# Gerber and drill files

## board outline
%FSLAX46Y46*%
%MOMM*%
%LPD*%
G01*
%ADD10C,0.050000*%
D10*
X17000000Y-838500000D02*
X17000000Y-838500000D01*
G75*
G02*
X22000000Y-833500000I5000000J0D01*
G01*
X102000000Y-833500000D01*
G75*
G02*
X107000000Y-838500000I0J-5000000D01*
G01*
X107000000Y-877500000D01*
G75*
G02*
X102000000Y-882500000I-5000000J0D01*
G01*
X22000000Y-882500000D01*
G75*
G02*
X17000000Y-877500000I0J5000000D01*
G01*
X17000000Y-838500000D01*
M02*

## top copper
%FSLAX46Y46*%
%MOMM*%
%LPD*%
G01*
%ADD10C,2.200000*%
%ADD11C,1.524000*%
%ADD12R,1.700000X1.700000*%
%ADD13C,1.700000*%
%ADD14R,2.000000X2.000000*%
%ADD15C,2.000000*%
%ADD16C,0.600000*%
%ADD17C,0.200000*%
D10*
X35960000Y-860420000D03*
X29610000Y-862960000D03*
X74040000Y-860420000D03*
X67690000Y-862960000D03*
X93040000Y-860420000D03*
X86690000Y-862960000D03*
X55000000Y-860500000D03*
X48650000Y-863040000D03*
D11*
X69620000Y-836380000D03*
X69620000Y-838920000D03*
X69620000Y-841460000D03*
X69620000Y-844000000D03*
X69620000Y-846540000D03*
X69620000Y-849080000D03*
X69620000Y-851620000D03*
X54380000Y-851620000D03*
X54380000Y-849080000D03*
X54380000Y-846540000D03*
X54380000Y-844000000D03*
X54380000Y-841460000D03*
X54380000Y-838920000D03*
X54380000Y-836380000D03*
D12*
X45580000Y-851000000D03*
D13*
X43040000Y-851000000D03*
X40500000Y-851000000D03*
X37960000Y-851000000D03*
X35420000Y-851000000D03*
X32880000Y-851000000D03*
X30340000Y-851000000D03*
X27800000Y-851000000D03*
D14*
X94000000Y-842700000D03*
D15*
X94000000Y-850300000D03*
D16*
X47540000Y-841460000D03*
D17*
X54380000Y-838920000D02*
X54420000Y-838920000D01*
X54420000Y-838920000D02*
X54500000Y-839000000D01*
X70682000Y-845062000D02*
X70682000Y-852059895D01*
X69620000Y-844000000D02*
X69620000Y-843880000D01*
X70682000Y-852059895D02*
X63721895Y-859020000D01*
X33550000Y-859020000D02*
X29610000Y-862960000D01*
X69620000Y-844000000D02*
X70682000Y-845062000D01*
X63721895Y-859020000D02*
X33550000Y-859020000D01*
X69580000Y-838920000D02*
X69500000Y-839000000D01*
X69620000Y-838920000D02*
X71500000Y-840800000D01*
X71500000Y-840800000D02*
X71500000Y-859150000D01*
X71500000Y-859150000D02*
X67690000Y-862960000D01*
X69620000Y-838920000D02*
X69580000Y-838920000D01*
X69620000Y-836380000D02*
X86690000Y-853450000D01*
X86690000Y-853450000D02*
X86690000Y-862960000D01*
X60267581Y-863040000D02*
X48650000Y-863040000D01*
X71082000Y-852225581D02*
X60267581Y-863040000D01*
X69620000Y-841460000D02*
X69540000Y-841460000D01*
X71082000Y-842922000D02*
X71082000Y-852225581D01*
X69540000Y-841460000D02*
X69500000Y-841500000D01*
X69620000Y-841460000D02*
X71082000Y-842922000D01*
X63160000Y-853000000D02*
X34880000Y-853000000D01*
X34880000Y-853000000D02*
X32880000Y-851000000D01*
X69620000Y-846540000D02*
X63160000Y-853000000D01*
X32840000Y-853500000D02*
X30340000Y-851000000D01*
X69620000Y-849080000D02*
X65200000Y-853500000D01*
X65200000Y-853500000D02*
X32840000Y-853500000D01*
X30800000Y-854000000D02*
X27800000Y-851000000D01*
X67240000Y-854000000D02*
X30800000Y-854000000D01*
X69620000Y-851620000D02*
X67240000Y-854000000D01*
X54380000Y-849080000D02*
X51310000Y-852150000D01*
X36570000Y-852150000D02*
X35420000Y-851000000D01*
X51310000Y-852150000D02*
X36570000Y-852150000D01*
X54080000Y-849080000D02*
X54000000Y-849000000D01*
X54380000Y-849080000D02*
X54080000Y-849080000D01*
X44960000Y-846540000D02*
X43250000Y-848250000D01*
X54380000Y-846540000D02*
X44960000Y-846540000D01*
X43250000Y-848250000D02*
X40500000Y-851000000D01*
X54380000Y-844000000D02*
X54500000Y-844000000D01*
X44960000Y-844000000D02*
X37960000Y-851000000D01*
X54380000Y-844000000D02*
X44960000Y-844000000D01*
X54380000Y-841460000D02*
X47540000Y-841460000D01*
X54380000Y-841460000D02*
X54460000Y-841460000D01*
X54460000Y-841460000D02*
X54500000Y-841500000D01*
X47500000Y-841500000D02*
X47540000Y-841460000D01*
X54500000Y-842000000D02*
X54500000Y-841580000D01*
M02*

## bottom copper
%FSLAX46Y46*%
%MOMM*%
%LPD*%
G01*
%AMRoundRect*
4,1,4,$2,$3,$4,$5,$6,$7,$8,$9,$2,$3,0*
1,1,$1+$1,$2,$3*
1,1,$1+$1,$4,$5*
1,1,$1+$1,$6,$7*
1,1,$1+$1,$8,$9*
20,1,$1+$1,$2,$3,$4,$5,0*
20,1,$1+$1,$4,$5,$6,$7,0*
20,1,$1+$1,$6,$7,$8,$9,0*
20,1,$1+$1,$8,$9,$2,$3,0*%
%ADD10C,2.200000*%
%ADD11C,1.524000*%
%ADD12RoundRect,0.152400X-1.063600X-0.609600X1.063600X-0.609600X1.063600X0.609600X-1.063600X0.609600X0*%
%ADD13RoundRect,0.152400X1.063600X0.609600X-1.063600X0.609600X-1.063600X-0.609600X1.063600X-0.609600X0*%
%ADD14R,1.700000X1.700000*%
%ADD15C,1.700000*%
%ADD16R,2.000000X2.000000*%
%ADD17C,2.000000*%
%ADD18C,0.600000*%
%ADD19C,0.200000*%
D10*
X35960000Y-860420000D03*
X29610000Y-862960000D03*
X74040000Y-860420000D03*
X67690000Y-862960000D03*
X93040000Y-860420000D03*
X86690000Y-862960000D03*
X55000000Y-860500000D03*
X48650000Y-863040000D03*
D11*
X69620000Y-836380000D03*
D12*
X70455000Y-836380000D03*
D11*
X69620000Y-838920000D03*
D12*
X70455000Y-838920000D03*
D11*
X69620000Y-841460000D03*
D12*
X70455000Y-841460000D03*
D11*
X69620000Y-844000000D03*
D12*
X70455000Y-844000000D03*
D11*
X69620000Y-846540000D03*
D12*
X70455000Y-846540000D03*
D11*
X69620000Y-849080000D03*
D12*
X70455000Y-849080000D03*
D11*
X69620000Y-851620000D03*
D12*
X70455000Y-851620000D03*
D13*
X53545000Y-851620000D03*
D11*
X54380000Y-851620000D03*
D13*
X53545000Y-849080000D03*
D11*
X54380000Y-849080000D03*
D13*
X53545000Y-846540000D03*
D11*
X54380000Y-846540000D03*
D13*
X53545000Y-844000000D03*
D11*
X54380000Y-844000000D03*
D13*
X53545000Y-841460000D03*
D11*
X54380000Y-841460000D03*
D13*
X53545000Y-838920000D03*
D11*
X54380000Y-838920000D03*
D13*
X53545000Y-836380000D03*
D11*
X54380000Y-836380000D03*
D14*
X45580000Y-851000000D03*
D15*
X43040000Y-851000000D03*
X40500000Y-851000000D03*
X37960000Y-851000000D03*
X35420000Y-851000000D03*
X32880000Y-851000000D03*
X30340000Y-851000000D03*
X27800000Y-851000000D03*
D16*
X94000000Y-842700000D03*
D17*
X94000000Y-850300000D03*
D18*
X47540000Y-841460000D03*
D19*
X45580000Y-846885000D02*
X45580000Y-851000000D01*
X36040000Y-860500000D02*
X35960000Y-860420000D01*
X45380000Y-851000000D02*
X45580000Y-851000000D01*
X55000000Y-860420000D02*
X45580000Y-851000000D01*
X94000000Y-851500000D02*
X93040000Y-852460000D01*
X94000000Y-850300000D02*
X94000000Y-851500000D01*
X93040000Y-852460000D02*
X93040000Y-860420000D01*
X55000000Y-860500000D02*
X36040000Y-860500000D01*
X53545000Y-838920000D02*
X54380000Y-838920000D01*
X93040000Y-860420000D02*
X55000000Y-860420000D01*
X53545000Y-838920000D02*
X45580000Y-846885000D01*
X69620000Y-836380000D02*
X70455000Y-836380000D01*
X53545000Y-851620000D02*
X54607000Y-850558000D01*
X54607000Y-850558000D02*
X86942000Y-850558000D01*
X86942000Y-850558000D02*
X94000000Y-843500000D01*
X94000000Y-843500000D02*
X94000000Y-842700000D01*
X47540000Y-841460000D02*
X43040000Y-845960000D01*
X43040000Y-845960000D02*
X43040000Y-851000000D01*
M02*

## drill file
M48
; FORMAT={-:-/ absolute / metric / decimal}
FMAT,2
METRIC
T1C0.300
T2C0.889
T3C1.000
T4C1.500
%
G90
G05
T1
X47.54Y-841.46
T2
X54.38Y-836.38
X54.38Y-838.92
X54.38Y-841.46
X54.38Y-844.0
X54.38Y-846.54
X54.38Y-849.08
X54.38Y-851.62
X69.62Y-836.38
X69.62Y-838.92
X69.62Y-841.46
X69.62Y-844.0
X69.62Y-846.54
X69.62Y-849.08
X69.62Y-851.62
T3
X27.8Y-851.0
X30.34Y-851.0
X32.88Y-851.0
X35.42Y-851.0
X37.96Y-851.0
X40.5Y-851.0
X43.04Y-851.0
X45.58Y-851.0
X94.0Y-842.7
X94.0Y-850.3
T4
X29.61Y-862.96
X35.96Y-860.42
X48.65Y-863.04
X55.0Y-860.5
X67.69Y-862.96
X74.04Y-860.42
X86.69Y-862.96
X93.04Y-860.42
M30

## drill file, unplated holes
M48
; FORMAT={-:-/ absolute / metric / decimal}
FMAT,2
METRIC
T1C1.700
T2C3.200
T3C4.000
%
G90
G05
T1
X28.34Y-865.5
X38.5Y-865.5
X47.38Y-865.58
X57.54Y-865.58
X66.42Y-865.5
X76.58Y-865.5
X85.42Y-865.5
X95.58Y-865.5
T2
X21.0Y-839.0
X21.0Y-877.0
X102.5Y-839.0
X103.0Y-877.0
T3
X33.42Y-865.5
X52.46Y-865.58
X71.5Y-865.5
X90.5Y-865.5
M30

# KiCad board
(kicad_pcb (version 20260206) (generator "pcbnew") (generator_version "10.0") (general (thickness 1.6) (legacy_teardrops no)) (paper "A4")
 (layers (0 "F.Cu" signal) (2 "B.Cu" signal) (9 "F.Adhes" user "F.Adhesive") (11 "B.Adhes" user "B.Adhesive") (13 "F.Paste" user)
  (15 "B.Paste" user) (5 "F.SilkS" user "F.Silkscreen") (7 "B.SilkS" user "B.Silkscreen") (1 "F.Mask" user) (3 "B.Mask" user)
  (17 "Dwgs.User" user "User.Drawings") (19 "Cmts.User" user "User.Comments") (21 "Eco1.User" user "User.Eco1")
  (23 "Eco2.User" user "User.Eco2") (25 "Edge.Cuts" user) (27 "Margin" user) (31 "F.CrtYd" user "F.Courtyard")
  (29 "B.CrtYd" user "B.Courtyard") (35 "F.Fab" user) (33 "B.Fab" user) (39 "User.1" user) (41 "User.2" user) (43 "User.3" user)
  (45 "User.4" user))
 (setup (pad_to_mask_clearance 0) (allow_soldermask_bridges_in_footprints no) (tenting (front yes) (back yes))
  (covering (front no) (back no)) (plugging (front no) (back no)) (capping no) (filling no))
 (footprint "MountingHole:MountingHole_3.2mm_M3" (layer "F.Cu") (at 21 877)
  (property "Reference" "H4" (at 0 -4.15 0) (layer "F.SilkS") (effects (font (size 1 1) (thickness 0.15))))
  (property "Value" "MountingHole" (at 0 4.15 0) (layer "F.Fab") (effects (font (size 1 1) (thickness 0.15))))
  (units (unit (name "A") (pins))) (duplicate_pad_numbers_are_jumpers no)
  (pad "" np_thru_hole circle (at 0 0) (size 3.2 3.2) (drill 3.2) (layers "*.Cu" "*.Mask")))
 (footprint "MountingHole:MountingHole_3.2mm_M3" (layer "F.Cu") (at 102.5 839)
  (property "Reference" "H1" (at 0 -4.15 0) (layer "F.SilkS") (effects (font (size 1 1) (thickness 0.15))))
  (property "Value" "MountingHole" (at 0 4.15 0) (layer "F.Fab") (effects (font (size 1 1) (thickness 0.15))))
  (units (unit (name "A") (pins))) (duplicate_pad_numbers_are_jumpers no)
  (pad "" np_thru_hole circle (at 0 0) (size 3.2 3.2) (drill 3.2) (layers "*.Cu" "*.Mask")))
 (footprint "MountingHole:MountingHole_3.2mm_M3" (layer "F.Cu") (at 21 839)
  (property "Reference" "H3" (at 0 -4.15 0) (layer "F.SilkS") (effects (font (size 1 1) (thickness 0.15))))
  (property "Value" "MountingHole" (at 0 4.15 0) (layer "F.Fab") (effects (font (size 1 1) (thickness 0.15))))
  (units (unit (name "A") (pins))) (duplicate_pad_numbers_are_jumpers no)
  (pad "" np_thru_hole circle (at 0 0) (size 3.2 3.2) (drill 3.2) (layers "*.Cu" "*.Mask")))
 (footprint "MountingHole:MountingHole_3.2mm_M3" (layer "F.Cu") (at 103 877)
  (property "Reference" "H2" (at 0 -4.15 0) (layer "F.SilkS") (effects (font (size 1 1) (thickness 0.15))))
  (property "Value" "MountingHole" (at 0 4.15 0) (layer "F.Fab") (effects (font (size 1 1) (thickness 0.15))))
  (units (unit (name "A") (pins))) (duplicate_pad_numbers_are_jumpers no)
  (pad "" np_thru_hole circle (at 0 0) (size 3.2 3.2) (drill 3.2) (layers "*.Cu" "*.Mask")))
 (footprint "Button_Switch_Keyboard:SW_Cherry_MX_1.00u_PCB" (layer "F.Cu") (at 35.96 860.42)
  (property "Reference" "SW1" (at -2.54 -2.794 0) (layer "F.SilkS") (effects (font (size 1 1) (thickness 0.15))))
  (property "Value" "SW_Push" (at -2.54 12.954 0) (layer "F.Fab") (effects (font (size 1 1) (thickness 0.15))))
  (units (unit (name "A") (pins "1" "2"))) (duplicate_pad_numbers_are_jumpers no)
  (pad "" np_thru_hole circle (at -7.62 5.08) (size 1.7 1.7) (drill 1.7) (layers "*.Cu" "*.Mask"))
  (pad "" np_thru_hole circle (at -2.54 5.08) (size 4 4) (drill 4) (layers "*.Cu" "*.Mask"))
  (pad "" np_thru_hole circle (at 2.54 5.08) (size 1.7 1.7) (drill 1.7) (layers "*.Cu" "*.Mask"))
  (pad "1" thru_hole circle (at 0 0) (size 2.2 2.2) (drill 1.5) (layers "*.Cu" "*.Mask") (remove_unused_layers no) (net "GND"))
  (pad "2" thru_hole circle (at -6.35 2.54) (size 2.2 2.2) (drill 1.5) (layers "*.Cu" "*.Mask") (remove_unused_layers no)
   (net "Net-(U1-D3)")))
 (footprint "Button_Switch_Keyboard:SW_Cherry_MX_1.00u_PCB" (layer "F.Cu") (at 74.04 860.42)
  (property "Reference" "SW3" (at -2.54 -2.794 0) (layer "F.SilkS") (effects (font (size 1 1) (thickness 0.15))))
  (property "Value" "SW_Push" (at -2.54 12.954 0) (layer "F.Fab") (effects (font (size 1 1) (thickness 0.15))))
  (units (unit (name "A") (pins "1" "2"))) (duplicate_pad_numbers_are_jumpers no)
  (pad "" np_thru_hole circle (at -7.62 5.08) (size 1.7 1.7) (drill 1.7) (layers "*.Cu" "*.Mask"))
  (pad "" np_thru_hole circle (at -2.54 5.08) (size 4 4) (drill 4) (layers "*.Cu" "*.Mask"))
  (pad "" np_thru_hole circle (at 2.54 5.08) (size 1.7 1.7) (drill 1.7) (layers "*.Cu" "*.Mask"))
  (pad "1" thru_hole circle (at 0 0) (size 2.2 2.2) (drill 1.5) (layers "*.Cu" "*.Mask") (remove_unused_layers no) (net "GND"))
  (pad "2" thru_hole circle (at -6.35 2.54) (size 2.2 2.2) (drill 1.5) (layers "*.Cu" "*.Mask") (remove_unused_layers no)
   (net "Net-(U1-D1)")))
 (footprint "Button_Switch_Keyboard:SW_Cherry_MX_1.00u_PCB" (layer "F.Cu") (at 93.04 860.42)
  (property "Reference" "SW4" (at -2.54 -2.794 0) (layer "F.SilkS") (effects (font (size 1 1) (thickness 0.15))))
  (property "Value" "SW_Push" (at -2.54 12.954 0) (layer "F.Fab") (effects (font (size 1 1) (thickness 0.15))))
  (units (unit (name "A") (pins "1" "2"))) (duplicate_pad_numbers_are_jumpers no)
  (pad "" np_thru_hole circle (at -7.62 5.08) (size 1.7 1.7) (drill 1.7) (layers "*.Cu" "*.Mask"))
  (pad "" np_thru_hole circle (at -2.54 5.08) (size 4 4) (drill 4) (layers "*.Cu" "*.Mask"))
  (pad "" np_thru_hole circle (at 2.54 5.08) (size 1.7 1.7) (drill 1.7) (layers "*.Cu" "*.Mask"))
  (pad "1" thru_hole circle (at 0 0) (size 2.2 2.2) (drill 1.5) (layers "*.Cu" "*.Mask") (remove_unused_layers no) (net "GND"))
  (pad "2" thru_hole circle (at -6.35 2.54) (size 2.2 2.2) (drill 1.5) (layers "*.Cu" "*.Mask") (remove_unused_layers no)
   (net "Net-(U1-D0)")))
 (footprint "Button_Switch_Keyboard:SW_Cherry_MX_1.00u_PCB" (layer "F.Cu") (at 55 860.5)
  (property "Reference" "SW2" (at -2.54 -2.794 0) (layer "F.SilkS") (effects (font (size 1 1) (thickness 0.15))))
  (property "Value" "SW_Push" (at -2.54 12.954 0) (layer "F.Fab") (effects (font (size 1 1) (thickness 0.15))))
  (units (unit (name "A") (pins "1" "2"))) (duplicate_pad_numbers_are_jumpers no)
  (pad "" np_thru_hole circle (at -7.62 5.08) (size 1.7 1.7) (drill 1.7) (layers "*.Cu" "*.Mask"))
  (pad "" np_thru_hole circle (at -2.54 5.08) (size 4 4) (drill 4) (layers "*.Cu" "*.Mask"))
  (pad "" np_thru_hole circle (at 2.54 5.08) (size 1.7 1.7) (drill 1.7) (layers "*.Cu" "*.Mask"))
  (pad "1" thru_hole circle (at 0 0) (size 2.2 2.2) (drill 1.5) (layers "*.Cu" "*.Mask") (remove_unused_layers no) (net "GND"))
  (pad "2" thru_hole circle (at -6.35 2.54) (size 2.2 2.2) (drill 1.5) (layers "*.Cu" "*.Mask") (remove_unused_layers no)
   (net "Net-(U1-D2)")))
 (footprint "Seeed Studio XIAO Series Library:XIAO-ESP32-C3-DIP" (layer "B.Cu") (at 62 844 90)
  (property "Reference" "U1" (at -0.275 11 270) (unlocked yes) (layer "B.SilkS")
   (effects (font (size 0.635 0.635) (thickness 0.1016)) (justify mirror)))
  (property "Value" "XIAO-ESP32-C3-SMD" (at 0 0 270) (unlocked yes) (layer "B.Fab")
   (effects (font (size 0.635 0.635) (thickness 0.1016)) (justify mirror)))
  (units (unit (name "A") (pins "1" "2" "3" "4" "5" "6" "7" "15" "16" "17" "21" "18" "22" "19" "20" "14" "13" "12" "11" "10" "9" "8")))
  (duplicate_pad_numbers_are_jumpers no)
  (pad "1" thru_hole circle (at 7.62 7.62) (size 1.524 1.524) (drill 0.889) (layers "*.Cu" "*.Mask") (remove_unused_layers no)
   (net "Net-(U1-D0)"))
  (pad "1" smd roundrect (at 7.62 8.455) (size 2.432 1.524) (layers "B.Cu" "B.Mask") (roundrect_rratio 0.1) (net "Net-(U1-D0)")
   (thermal_bridge_angle 45))
  (pad "2" thru_hole circle (at 5.08 7.62) (size 1.524 1.524) (drill 0.889) (layers "*.Cu" "*.Mask") (remove_unused_layers no)
   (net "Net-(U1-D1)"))
  (pad "2" smd roundrect (at 5.08 8.455) (size 2.432 1.524) (layers "B.Cu" "B.Mask") (roundrect_rratio 0.1) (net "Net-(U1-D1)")
   (thermal_bridge_angle 45))
  (pad "3" thru_hole circle (at 2.54 7.62) (size 1.524 1.524) (drill 0.889) (layers "*.Cu" "*.Mask") (remove_unused_layers no)
   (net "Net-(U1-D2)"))
  (pad "3" smd roundrect (at 2.54 8.455) (size 2.432 1.524) (layers "B.Cu" "B.Mask") (roundrect_rratio 0.1) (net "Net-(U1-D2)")
   (thermal_bridge_angle 45))
  (pad "4" thru_hole circle (at 0 7.62) (size 1.524 1.524) (drill 0.889) (layers "*.Cu" "*.Mask") (remove_unused_layers no)
   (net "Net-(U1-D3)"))
  (pad "4" smd roundrect (at 0 8.455) (size 2.432 1.524) (layers "B.Cu" "B.Mask") (roundrect_rratio 0.1) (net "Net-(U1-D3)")
   (thermal_bridge_angle 45))
  (pad "5" thru_hole circle (at -2.54 7.62) (size 1.524 1.524) (drill 0.889) (layers "*.Cu" "*.Mask") (remove_unused_layers no) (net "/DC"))
  (pad "5" smd roundrect (at -2.54 8.455) (size 2.432 1.524) (layers "B.Cu" "B.Mask") (roundrect_rratio 0.1) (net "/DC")
   (thermal_bridge_angle 45))
  (pad "6" thru_hole circle (at -5.08 7.62) (size 1.524 1.524) (drill 0.889) (layers "*.Cu" "*.Mask") (remove_unused_layers no) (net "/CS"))
  (pad "6" smd roundrect (at -5.08 8.455) (size 2.432 1.524) (layers "B.Cu" "B.Mask") (roundrect_rratio 0.1) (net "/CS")
   (thermal_bridge_angle 45))
  (pad "7" thru_hole circle (at -7.62 7.62) (size 1.524 1.524) (drill 0.889) (layers "*.Cu" "*.Mask") (remove_unused_layers no) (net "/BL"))
  (pad "7" smd roundrect (at -7.62 8.455) (size 2.432 1.524) (layers "B.Cu" "B.Mask") (roundrect_rratio 0.1) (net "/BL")
   (thermal_bridge_angle 45))
  (pad "8" smd roundrect (at -7.62 -8.455 180) (size 2.432 1.524) (layers "B.Cu" "B.Mask") (roundrect_rratio 0.1) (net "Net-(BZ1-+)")
   (thermal_bridge_angle 45))
  (pad "8" thru_hole circle (at -7.62 -7.62 180) (size 1.524 1.524) (drill 0.889) (layers "*.Cu" "*.Mask") (remove_unused_layers no)
   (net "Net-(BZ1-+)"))
  (pad "9" smd roundrect (at -5.08 -8.455 180) (size 2.432 1.524) (layers "B.Cu" "B.Mask") (roundrect_rratio 0.1) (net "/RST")
   (thermal_bridge_angle 45))
  (pad "9" thru_hole circle (at -5.08 -7.62 180) (size 1.524 1.524) (drill 0.889) (layers "*.Cu" "*.Mask") (remove_unused_layers no)
   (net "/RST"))
  (pad "10" smd roundrect (at -2.54 -8.455 180) (size 2.432 1.524) (layers "B.Cu" "B.Mask") (roundrect_rratio 0.1) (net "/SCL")
   (thermal_bridge_angle 45))
  (pad "10" thru_hole circle (at -2.54 -7.62 180) (size 1.524 1.524) (drill 0.889) (layers "*.Cu" "*.Mask") (remove_unused_layers no)
   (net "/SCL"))
  (pad "11" smd roundrect (at 0 -8.455 180) (size 2.432 1.524) (layers "B.Cu" "B.Mask") (roundrect_rratio 0.1) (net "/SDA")
   (thermal_bridge_angle 45))
  (pad "11" thru_hole circle (at 0 -7.62 180) (size 1.524 1.524) (drill 0.889) (layers "*.Cu" "*.Mask") (remove_unused_layers no)
   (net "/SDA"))
  (pad "12" smd roundrect (at 2.54 -8.455 180) (size 2.432 1.524) (layers "B.Cu" "B.Mask") (roundrect_rratio 0.1) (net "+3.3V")
   (thermal_bridge_angle 45))
  (pad "12" thru_hole circle (at 2.54 -7.62 180) (size 1.524 1.524) (drill 0.889) (layers "*.Cu" "*.Mask") (remove_unused_layers no)
   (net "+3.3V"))
  (pad "13" smd roundrect (at 5.08 -8.455 180) (size 2.432 1.524) (layers "B.Cu" "B.Mask") (roundrect_rratio 0.1) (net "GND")
   (thermal_bridge_angle 45))
  (pad "13" thru_hole circle (at 5.08 -7.62 180) (size 1.524 1.524) (drill 0.889) (layers "*.Cu" "*.Mask") (remove_unused_layers no)
   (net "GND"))
  (pad "14" smd roundrect (at 7.62 -8.455 180) (size 2.432 1.524) (layers "B.Cu" "B.Mask") (roundrect_rratio 0.1)
   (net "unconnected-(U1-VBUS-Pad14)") (thermal_bridge_angle 45))
  (pad "14" thru_hole circle (at 7.62 -7.62 180) (size 1.524 1.524) (drill 0.889) (layers "*.Cu" "*.Mask") (remove_unused_layers no)
   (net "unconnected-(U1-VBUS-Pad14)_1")))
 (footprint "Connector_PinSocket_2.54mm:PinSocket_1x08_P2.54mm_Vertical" (layer "B.Cu") (at 45.58 851 90)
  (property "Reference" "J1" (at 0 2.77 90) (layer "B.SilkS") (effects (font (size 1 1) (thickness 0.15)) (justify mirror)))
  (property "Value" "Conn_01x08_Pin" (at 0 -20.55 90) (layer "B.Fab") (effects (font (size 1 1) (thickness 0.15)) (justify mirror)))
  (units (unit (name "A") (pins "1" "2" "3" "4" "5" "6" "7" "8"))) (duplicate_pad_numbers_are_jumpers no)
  (pad "1" thru_hole rect (at 0 0 90) (size 1.7 1.7) (drill 1) (layers "*.Cu" "*.Mask") (remove_unused_layers no) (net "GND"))
  (pad "2" thru_hole circle (at 0 -2.54 90) (size 1.7 1.7) (drill 1) (layers "*.Cu" "*.Mask") (remove_unused_layers no) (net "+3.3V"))
  (pad "3" thru_hole circle (at 0 -5.08 90) (size 1.7 1.7) (drill 1) (layers "*.Cu" "*.Mask") (remove_unused_layers no) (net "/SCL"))
  (pad "4" thru_hole circle (at 0 -7.62 90) (size 1.7 1.7) (drill 1) (layers "*.Cu" "*.Mask") (remove_unused_layers no) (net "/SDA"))
  (pad "5" thru_hole circle (at 0 -10.16 90) (size 1.7 1.7) (drill 1) (layers "*.Cu" "*.Mask") (remove_unused_layers no) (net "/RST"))
  (pad "6" thru_hole circle (at 0 -12.7 90) (size 1.7 1.7) (drill 1) (layers "*.Cu" "*.Mask") (remove_unused_layers no) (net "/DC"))
  (pad "7" thru_hole circle (at 0 -15.24 90) (size 1.7 1.7) (drill 1) (layers "*.Cu" "*.Mask") (remove_unused_layers no) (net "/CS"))
  (pad "8" thru_hole circle (at 0 -17.78 90) (size 1.7 1.7) (drill 1) (layers "*.Cu" "*.Mask") (remove_unused_layers no) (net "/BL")))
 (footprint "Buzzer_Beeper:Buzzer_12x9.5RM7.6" (layer "B.Cu") (at 94 842.7 -90)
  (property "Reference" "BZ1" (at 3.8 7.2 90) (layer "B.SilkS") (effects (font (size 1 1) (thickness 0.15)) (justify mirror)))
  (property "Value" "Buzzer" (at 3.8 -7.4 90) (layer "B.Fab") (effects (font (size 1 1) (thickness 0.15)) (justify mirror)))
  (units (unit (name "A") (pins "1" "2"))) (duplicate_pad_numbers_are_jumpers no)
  (pad "1" thru_hole rect (at 0 0 270) (size 2 2) (drill 1) (layers "*.Cu" "*.Mask") (remove_unused_layers no) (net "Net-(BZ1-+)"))
  (pad "2" thru_hole circle (at 7.6 0 270) (size 2 2) (drill 1) (layers "*.Cu" "*.Mask") (remove_unused_layers no) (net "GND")))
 (gr_rect (start 17 833.5) (end 107 882.5) (radius 5) (stroke (width 0.05) (type solid)) (fill no) (layer "Edge.Cuts"))
 (segment (start 54.38 838.92) (end 54.42 838.92) (width 0.2) (layer "F.Cu") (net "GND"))
 (segment (start 54.42 838.92) (end 54.5 839) (width 0.2) (layer "F.Cu") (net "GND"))
 (segment (start 45.58 846.885) (end 45.58 851) (width 0.2) (layer "B.Cu") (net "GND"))
 (segment (start 36.04 860.5) (end 35.96 860.42) (width 0.2) (layer "B.Cu") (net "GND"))
 (segment (start 45.38 851) (end 45.58 851) (width 0.2) (layer "B.Cu") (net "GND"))
 (segment (start 55 860.42) (end 45.58 851) (width 0.2) (layer "B.Cu") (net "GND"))
 (segment (start 94 851.5) (end 93.04 852.46) (width 0.2) (layer "B.Cu") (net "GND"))
 (segment (start 94 850.3) (end 94 851.5) (width 0.2) (layer "B.Cu") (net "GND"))
 (segment (start 93.04 852.46) (end 93.04 860.42) (width 0.2) (layer "B.Cu") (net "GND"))
 (segment (start 55 860.5) (end 36.04 860.5) (width 0.2) (layer "B.Cu") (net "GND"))
 (segment (start 53.545 838.92) (end 54.38 838.92) (width 0.2) (layer "B.Cu") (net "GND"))
 (segment (start 93.04 860.42) (end 55 860.42) (width 0.2) (layer "B.Cu") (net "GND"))
 (segment (start 53.545 838.92) (end 45.58 846.885) (width 0.2) (layer "B.Cu") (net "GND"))
 (segment (start 70.682 845.062) (end 70.682 852.059895) (width 0.2) (layer "F.Cu") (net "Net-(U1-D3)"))
 (segment (start 69.62 844) (end 69.62 843.88) (width 0.2) (layer "F.Cu") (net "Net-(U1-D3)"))
 (segment (start 70.682 852.059895) (end 63.721895 859.02) (width 0.2) (layer "F.Cu") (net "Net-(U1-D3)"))
 (segment (start 33.55 859.02) (end 29.61 862.96) (width 0.2) (layer "F.Cu") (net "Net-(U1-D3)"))
 (segment (start 69.62 844) (end 70.682 845.062) (width 0.2) (layer "F.Cu") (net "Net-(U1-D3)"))
 (segment (start 63.721895 859.02) (end 33.55 859.02) (width 0.2) (layer "F.Cu") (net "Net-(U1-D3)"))
 (segment (start 69.58 838.92) (end 69.5 839) (width 0.2) (layer "F.Cu") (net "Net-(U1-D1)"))
 (segment (start 69.62 838.92) (end 71.5 840.8) (width 0.2) (layer "F.Cu") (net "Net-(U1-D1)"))
 (segment (start 71.5 840.8) (end 71.5 859.15) (width 0.2) (layer "F.Cu") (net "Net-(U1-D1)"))
 (segment (start 71.5 859.15) (end 67.69 862.96) (width 0.2) (layer "F.Cu") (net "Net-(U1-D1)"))
 (segment (start 69.62 838.92) (end 69.58 838.92) (width 0.2) (layer "F.Cu") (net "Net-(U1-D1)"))
 (segment (start 69.62 836.38) (end 86.69 853.45) (width 0.2) (layer "F.Cu") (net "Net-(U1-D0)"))
 (segment (start 86.69 853.45) (end 86.69 862.96) (width 0.2) (layer "F.Cu") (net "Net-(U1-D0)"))
 (segment (start 69.62 836.38) (end 70.455 836.38) (width 0.2) (layer "B.Cu") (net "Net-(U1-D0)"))
 (segment (start 60.267581 863.04) (end 48.65 863.04) (width 0.2) (layer "F.Cu") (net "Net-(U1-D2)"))
 (segment (start 71.082 852.225581) (end 60.267581 863.04) (width 0.2) (layer "F.Cu") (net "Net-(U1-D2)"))
 (segment (start 69.62 841.46) (end 69.54 841.46) (width 0.2) (layer "F.Cu") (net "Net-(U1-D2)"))
 (segment (start 71.082 842.922) (end 71.082 852.225581) (width 0.2) (layer "F.Cu") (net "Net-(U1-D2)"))
 (segment (start 69.54 841.46) (end 69.5 841.5) (width 0.2) (layer "F.Cu") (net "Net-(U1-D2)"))
 (segment (start 69.62 841.46) (end 71.082 842.922) (width 0.2) (layer "F.Cu") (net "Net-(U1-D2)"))
 (segment (start 63.16 853) (end 34.88 853) (width 0.2) (layer "F.Cu") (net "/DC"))
 (segment (start 34.88 853) (end 32.88 851) (width 0.2) (layer "F.Cu") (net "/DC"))
 (segment (start 69.62 846.54) (end 63.16 853) (width 0.2) (layer "F.Cu") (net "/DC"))
 (segment (start 32.84 853.5) (end 30.34 851) (width 0.2) (layer "F.Cu") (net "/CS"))
 (segment (start 69.62 849.08) (end 65.2 853.5) (width 0.2) (layer "F.Cu") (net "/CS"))
 (segment (start 65.2 853.5) (end 32.84 853.5) (width 0.2) (layer "F.Cu") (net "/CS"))
 (segment (start 30.8 854) (end 27.8 851) (width 0.2) (layer "F.Cu") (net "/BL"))
 (segment (start 67.24 854) (end 30.8 854) (width 0.2) (layer "F.Cu") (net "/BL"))
 (segment (start 69.62 851.62) (end 67.24 854) (width 0.2) (layer "F.Cu") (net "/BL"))
 (segment (start 53.545 851.62) (end 54.607 850.558) (width 0.2) (layer "B.Cu") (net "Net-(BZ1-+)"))
 (segment (start 54.607 850.558) (end 86.942 850.558) (width 0.2) (layer "B.Cu") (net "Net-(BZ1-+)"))
 (segment (start 86.942 850.558) (end 94 843.5) (width 0.2) (layer "B.Cu") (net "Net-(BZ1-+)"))
 (segment (start 94 843.5) (end 94 842.7) (width 0.2) (layer "B.Cu") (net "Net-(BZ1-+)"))
 (segment (start 54.38 849.08) (end 51.31 852.15) (width 0.2) (layer "F.Cu") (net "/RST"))
 (segment (start 36.57 852.15) (end 35.42 851) (width 0.2) (layer "F.Cu") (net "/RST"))
 (segment (start 51.31 852.15) (end 36.57 852.15) (width 0.2) (layer "F.Cu") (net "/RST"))
 (segment (start 54.08 849.08) (end 54 849) (width 0.2) (layer "F.Cu") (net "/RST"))
 (segment (start 54.38 849.08) (end 54.08 849.08) (width 0.2) (layer "F.Cu") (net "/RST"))
 (segment (start 44.96 846.54) (end 43.25 848.25) (width 0.2) (layer "F.Cu") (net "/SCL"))
 (segment (start 54.38 846.54) (end 44.96 846.54) (width 0.2) (layer "F.Cu") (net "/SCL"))
 (segment (start 43.25 848.25) (end 40.5 851) (width 0.2) (layer "F.Cu") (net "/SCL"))
 (segment (start 54.38 844) (end 54.5 844) (width 0.2) (layer "F.Cu") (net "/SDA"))
 (segment (start 44.96 844) (end 37.96 851) (width 0.2) (layer "F.Cu") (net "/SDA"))
 (segment (start 54.38 844) (end 44.96 844) (width 0.2) (layer "F.Cu") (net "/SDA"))
 (segment (start 54.38 841.46) (end 47.54 841.46) (width 0.2) (layer "F.Cu") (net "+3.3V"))
 (segment (start 54.38 841.46) (end 54.46 841.46) (width 0.2) (layer "F.Cu") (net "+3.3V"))
 (segment (start 54.46 841.46) (end 54.5 841.5) (width 0.2) (layer "F.Cu") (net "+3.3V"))
 (segment (start 47.5 841.5) (end 47.54 841.46) (width 0.2) (layer "F.Cu") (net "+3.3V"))
 (segment (start 54.5 842) (end 54.5 841.58) (width 0.2) (layer "F.Cu") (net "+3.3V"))
 (via (at 47.54 841.46) (size 0.6) (drill 0.3) (layers "F.Cu" "B.Cu") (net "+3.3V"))
 (segment (start 47.54 841.46) (end 43.04 845.96) (width 0.2) (layer "B.Cu") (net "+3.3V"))
 (segment (start 43.04 845.96) (end 43.04 851) (width 0.2) (layer "B.Cu") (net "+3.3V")))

